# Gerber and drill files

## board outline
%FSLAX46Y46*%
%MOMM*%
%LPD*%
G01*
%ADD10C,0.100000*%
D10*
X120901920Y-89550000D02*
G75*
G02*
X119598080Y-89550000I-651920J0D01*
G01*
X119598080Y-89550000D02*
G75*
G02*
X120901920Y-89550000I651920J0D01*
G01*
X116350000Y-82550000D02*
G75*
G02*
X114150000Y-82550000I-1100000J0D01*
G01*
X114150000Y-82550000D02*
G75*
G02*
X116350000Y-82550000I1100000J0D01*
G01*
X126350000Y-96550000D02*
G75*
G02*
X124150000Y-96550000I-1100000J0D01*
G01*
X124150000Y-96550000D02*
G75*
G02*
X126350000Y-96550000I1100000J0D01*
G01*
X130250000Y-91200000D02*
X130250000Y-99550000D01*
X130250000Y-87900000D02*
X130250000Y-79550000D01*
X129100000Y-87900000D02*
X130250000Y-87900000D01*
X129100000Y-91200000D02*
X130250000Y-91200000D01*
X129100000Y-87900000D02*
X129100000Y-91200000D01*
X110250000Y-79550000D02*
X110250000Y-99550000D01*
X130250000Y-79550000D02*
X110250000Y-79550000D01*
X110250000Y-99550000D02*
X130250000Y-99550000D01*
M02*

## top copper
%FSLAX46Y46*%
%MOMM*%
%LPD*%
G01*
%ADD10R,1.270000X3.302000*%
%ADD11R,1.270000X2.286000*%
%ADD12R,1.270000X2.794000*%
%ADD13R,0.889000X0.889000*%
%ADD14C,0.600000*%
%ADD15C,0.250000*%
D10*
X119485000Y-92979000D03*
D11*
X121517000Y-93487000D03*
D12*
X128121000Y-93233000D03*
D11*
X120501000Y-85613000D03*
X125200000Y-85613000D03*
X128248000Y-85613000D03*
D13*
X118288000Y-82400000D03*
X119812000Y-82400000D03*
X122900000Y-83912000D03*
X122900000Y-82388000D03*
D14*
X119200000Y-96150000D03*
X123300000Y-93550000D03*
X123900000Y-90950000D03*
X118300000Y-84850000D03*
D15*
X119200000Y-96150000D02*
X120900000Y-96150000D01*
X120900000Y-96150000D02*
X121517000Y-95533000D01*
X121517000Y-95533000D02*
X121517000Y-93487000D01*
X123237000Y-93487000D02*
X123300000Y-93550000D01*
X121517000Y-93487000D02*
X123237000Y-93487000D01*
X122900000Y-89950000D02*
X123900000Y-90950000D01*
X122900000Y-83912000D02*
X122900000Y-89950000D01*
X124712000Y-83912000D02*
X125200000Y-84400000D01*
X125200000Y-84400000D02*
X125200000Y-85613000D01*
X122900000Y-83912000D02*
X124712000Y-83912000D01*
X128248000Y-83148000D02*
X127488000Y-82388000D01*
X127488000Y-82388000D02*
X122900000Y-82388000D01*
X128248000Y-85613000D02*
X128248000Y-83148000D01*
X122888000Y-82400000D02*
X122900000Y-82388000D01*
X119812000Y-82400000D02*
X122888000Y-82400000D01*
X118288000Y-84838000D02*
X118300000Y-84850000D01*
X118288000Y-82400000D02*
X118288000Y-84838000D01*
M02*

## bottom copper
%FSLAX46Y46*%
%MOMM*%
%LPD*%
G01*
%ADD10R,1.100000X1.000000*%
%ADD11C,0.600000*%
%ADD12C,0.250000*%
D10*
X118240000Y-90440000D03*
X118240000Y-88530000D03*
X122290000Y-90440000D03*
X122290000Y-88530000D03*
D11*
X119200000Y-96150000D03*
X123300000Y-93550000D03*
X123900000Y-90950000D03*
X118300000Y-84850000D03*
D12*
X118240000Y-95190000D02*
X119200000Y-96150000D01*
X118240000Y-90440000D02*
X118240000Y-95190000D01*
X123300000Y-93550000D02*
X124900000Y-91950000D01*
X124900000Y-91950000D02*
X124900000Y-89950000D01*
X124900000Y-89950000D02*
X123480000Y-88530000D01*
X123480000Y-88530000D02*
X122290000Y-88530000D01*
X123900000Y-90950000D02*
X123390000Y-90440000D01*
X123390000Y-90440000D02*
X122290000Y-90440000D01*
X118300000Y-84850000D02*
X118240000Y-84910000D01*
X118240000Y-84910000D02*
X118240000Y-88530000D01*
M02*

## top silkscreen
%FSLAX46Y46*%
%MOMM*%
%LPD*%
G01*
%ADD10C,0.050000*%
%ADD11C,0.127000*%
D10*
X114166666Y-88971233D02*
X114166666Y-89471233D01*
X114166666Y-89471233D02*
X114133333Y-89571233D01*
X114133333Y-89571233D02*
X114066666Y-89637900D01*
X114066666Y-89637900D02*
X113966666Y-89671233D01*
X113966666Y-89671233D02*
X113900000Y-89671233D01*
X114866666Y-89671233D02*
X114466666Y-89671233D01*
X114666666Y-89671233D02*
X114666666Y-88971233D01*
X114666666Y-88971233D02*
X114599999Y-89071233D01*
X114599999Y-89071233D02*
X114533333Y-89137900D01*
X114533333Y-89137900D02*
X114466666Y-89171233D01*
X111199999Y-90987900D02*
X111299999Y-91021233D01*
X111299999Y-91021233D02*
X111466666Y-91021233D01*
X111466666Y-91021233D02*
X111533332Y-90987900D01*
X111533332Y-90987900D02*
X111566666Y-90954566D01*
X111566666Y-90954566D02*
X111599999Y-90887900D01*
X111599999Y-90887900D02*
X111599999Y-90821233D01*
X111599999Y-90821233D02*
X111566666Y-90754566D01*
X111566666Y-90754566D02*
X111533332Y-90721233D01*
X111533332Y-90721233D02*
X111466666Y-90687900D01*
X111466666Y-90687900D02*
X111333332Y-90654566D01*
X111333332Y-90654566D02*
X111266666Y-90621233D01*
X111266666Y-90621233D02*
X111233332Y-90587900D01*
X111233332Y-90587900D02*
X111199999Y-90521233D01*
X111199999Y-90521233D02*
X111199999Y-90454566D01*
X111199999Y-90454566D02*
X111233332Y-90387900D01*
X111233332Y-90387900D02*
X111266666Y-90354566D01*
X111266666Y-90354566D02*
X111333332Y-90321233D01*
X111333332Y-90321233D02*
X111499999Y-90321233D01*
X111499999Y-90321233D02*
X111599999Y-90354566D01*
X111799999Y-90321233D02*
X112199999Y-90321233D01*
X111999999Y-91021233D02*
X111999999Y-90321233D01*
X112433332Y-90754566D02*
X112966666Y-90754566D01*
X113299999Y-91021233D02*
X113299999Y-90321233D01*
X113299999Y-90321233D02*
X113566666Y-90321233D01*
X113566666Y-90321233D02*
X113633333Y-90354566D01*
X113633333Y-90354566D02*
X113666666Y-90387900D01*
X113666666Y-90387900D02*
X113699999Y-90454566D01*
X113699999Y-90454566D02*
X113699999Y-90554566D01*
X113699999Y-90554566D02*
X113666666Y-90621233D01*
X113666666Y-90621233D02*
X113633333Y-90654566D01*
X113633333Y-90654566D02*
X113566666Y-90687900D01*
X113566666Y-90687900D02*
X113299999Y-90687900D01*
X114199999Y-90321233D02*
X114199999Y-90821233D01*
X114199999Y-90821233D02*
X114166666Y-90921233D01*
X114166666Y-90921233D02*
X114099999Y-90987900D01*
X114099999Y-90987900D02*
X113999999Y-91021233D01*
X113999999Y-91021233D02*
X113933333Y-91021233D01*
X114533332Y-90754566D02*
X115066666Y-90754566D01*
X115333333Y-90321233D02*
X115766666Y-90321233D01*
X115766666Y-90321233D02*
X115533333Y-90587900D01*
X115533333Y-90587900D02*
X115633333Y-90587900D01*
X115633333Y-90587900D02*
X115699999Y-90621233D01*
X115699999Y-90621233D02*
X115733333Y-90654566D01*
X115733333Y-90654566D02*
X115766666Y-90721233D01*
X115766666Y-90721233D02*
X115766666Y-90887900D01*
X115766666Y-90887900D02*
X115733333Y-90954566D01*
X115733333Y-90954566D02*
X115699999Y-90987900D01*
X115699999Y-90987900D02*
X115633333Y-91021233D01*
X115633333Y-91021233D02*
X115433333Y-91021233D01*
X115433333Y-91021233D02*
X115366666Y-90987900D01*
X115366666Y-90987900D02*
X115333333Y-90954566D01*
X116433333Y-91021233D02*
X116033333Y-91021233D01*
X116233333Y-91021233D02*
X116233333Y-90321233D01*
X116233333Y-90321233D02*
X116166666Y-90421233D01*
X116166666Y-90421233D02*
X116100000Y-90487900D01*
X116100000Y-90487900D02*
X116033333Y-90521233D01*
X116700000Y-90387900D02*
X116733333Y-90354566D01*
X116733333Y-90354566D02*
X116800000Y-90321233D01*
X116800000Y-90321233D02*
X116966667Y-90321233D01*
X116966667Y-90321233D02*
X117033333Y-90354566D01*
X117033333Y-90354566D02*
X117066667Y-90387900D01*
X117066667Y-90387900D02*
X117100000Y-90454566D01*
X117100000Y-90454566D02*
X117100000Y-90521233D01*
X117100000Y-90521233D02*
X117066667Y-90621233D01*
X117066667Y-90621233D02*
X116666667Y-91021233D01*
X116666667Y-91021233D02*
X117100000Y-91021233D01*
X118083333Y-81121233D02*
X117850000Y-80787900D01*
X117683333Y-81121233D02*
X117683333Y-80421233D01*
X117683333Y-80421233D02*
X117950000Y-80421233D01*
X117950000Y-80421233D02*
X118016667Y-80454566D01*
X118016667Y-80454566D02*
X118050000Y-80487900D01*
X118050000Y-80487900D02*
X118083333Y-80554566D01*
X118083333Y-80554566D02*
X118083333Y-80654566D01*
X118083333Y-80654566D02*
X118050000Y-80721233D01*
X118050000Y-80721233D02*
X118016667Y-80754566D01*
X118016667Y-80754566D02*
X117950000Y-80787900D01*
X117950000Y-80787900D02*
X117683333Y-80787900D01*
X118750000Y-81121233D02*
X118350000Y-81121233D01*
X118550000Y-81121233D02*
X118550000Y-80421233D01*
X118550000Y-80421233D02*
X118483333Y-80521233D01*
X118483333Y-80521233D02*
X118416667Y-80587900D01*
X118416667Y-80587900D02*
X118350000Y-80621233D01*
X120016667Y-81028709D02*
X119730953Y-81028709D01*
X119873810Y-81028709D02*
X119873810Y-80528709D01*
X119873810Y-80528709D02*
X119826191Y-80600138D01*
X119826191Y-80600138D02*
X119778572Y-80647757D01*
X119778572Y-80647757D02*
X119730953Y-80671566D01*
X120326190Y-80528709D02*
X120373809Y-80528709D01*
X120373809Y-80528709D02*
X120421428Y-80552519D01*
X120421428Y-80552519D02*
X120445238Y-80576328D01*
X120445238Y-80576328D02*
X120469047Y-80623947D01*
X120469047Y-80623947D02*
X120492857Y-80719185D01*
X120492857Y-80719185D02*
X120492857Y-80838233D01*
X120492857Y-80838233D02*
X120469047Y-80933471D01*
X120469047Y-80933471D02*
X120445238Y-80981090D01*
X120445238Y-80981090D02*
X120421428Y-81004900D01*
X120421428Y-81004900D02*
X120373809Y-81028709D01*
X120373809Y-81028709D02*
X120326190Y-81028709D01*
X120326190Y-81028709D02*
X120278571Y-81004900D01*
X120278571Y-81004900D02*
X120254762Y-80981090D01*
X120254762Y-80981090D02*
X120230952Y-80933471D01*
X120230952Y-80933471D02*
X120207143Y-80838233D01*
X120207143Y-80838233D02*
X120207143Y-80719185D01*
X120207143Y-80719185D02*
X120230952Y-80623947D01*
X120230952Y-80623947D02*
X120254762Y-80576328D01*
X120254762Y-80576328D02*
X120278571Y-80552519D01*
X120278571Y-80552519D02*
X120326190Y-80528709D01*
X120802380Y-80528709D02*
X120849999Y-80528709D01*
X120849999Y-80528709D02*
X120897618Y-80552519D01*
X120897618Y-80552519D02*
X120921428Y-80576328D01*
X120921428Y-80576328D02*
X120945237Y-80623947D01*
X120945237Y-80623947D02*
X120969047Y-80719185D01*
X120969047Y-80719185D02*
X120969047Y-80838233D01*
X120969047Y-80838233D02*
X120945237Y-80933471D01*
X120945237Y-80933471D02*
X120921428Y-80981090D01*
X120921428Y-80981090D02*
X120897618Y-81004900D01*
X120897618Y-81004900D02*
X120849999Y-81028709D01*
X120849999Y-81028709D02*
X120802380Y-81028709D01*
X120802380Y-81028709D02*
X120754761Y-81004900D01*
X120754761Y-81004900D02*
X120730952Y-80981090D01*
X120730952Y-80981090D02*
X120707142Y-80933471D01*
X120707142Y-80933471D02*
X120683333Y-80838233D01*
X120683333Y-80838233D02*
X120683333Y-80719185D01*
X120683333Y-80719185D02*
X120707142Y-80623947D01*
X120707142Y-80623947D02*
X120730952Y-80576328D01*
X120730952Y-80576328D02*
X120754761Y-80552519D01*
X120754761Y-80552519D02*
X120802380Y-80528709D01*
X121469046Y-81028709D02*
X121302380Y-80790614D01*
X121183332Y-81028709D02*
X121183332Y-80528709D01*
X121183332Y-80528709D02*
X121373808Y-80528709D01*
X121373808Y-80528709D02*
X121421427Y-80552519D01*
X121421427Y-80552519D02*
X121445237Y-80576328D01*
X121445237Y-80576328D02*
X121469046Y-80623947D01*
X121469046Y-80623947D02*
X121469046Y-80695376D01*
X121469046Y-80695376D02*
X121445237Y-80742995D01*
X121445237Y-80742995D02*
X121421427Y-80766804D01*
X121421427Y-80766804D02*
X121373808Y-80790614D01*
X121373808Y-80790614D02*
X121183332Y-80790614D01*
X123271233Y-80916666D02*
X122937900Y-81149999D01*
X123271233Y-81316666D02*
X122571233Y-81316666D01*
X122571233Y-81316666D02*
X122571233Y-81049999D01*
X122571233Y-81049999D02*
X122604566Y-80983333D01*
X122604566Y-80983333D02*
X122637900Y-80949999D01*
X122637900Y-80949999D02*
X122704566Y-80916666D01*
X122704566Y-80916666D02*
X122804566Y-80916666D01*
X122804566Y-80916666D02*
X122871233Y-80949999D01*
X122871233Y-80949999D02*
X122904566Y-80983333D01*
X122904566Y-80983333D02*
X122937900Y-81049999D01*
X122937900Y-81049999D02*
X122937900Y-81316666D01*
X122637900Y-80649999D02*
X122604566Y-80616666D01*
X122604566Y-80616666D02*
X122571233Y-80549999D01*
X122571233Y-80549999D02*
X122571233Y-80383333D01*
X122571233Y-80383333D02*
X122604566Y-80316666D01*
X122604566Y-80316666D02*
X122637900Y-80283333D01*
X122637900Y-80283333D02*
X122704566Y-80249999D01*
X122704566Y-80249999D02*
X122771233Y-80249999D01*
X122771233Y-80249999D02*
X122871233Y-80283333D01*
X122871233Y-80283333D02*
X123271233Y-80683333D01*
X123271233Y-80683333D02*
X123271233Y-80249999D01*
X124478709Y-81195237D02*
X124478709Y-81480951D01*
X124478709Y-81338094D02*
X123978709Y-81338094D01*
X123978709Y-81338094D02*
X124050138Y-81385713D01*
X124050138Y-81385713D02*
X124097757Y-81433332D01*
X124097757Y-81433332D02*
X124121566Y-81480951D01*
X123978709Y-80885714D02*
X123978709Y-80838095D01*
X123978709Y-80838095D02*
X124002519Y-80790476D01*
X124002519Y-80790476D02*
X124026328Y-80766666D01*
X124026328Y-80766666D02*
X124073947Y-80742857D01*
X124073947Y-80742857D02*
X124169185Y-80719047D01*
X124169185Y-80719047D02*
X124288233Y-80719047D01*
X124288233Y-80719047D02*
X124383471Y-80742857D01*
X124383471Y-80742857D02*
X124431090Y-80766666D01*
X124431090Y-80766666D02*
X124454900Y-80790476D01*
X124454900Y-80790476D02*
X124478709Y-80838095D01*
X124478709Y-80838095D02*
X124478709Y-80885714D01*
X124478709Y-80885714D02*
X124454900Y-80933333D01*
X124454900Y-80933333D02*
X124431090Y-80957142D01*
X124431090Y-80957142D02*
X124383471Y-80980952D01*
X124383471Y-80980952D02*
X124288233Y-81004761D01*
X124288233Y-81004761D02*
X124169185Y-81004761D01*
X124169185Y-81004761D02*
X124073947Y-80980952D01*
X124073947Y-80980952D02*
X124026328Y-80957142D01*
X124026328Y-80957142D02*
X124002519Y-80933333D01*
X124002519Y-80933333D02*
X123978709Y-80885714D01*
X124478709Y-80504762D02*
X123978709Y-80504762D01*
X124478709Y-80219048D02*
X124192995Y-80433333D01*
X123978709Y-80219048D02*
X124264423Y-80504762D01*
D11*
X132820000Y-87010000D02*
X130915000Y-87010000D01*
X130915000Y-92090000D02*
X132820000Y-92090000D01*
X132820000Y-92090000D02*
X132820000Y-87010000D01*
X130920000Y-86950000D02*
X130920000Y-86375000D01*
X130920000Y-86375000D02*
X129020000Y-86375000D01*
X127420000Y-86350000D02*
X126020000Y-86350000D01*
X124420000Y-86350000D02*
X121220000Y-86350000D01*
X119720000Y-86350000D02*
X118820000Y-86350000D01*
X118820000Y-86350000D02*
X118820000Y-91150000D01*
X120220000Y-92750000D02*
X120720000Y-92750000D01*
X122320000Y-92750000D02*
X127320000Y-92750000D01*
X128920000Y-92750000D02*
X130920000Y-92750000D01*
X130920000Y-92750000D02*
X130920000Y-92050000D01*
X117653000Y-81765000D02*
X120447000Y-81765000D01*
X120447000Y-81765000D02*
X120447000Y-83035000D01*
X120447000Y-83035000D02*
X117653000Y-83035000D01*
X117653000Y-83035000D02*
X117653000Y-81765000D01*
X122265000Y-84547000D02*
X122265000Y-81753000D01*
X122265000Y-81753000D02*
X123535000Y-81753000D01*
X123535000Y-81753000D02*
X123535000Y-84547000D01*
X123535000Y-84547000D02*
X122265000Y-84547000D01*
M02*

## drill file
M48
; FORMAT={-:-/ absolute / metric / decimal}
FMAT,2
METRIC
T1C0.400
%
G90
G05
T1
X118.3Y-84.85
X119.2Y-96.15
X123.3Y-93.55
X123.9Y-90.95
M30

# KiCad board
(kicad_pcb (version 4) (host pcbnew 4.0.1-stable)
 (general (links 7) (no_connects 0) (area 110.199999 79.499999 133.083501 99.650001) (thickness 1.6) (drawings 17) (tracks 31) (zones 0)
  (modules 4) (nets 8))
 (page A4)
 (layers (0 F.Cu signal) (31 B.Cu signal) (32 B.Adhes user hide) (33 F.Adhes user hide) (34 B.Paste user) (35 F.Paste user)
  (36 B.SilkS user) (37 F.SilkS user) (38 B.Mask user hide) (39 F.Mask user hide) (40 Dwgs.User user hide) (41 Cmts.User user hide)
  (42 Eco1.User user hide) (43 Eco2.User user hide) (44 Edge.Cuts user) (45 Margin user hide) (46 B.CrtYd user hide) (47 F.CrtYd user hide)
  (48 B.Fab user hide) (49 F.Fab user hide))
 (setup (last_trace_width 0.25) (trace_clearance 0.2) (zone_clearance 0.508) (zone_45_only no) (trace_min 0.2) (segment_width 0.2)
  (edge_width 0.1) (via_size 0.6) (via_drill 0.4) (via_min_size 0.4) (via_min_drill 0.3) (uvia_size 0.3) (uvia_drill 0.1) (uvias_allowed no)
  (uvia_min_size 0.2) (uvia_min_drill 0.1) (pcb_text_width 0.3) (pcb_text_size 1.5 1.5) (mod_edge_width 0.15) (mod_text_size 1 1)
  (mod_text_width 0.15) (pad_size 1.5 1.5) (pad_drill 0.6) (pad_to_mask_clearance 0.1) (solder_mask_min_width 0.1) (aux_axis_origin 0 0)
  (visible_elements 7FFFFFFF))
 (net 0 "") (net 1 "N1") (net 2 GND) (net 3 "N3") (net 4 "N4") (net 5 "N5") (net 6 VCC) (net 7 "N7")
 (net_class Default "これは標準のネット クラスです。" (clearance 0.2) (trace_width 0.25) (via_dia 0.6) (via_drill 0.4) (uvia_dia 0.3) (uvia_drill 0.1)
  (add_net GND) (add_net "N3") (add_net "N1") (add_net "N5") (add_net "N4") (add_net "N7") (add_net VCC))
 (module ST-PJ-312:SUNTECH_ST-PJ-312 (layer F.Cu) (at 125.2 89.55) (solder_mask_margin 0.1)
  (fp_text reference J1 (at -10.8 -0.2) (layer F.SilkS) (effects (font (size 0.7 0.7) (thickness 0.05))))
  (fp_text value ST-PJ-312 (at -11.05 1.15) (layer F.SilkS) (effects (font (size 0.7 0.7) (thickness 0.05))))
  (fp_line (start 7.62 -2.54) (end 5.715 -2.54) (layer F.SilkS) (width 0.127))
  (fp_line (start 5.715 2.54) (end 7.62 2.54) (layer F.SilkS) (width 0.127))
  (fp_line (start 7.62 2.54) (end 7.62 -2.54) (layer F.SilkS) (width 0.127))
  (fp_line (start 5.72 -2.6) (end 5.72 -3.175) (layer F.SilkS) (width 0.127))
  (fp_line (start 5.72 -3.175) (end 3.82 -3.175) (layer F.SilkS) (width 0.127))
  (fp_line (start 2.22 -3.2) (end 0.82 -3.2) (layer F.SilkS) (width 0.127))
  (fp_line (start -0.78 -3.2) (end -3.98 -3.2) (layer F.SilkS) (width 0.127))
  (fp_line (start -5.48 -3.2) (end -6.38 -3.2) (layer F.SilkS) (width 0.127))
  (fp_line (start -6.38 -3.2) (end -6.38 1.6) (layer F.SilkS) (width 0.127))
  (fp_line (start -4.98 3.2) (end -4.48 3.2) (layer F.SilkS) (width 0.127))
  (fp_line (start -2.88 3.2) (end 2.12 3.2) (layer F.SilkS) (width 0.127))
  (fp_line (start 3.72 3.2) (end 5.72 3.2) (layer F.SilkS) (width 0.127))
  (fp_line (start 5.72 3.2) (end 5.72 2.5) (layer F.SilkS) (width 0.127))
  (pad LS smd rect (at -5.715 3.429 90) (size 3.302 1.27) (layers F.Cu F.Paste F.Mask) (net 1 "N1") (solder_mask_margin 0.2))
  (pad L smd rect (at -3.683 3.937 90) (size 2.286 1.27) (layers F.Cu F.Paste F.Mask) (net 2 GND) (solder_mask_margin 0.2))
  (pad COM2 smd rect (at 2.921 3.683 90) (size 2.794 1.27) (layers F.Cu F.Paste F.Mask) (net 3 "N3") (solder_mask_margin 0.2))
  (pad RS smd rect (at -4.699 -3.937 90) (size 2.286 1.27) (layers F.Cu F.Paste F.Mask) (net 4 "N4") (solder_mask_margin 0.2))
  (pad R smd rect (at 0 -3.937 90) (size 2.286 1.27) (layers F.Cu F.Paste F.Mask) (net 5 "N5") (solder_mask_margin 0.2))
  (pad COM1 smd rect (at 3.048 -3.937 90) (size 2.286 1.27) (layers F.Cu F.Paste F.Mask) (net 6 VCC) (solder_mask_margin 0.2)))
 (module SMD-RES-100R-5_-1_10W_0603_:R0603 (layer F.Cu) (at 119.05 82.4 90) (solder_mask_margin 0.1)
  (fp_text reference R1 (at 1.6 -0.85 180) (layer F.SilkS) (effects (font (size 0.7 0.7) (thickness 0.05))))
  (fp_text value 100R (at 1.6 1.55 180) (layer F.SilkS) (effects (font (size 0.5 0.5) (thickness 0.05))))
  (fp_line (start 0.635 -1.397) (end 0.635 1.397) (layer F.SilkS) (width 0.127))
  (fp_line (start 0.635 1.397) (end -0.635 1.397) (layer F.SilkS) (width 0.127))
  (fp_line (start -0.635 1.397) (end -0.635 -1.397) (layer F.SilkS) (width 0.127))
  (fp_line (start -0.635 -1.397) (end 0.635 -1.397) (layer F.SilkS) (width 0.127))
  (pad 1 smd rect (at 0 -0.762) (size 0.889 0.889) (layers F.Cu F.Paste F.Mask) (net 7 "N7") (solder_mask_margin 0.2))
  (pad 2 smd rect (at 0 0.762) (size 0.889 0.889) (layers F.Cu F.Paste F.Mask) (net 6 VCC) (solder_mask_margin 0.2)))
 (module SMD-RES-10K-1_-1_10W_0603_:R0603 (layer F.Cu) (at 122.9 83.15 180) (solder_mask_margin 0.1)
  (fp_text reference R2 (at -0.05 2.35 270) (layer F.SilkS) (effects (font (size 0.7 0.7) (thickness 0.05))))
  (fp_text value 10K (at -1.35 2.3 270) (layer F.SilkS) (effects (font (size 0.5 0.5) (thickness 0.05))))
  (fp_line (start 0.635 -1.397) (end 0.635 1.397) (layer F.SilkS) (width 0.127))
  (fp_line (start 0.635 1.397) (end -0.635 1.397) (layer F.SilkS) (width 0.127))
  (fp_line (start -0.635 1.397) (end -0.635 -1.397) (layer F.SilkS) (width 0.127))
  (fp_line (start -0.635 -1.397) (end 0.635 -1.397) (layer F.SilkS) (width 0.127))
  (pad 1 smd rect (at 0 -0.762 90) (size 0.889 0.889) (layers F.Cu F.Paste F.Mask) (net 5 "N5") (solder_mask_margin 0.2))
  (pad 2 smd rect (at 0 0.762 90) (size 0.889 0.889) (layers F.Cu F.Paste F.Mask) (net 6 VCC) (solder_mask_margin 0.2)))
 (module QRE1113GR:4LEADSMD (layer B.Cu) (at 120.25 89.5) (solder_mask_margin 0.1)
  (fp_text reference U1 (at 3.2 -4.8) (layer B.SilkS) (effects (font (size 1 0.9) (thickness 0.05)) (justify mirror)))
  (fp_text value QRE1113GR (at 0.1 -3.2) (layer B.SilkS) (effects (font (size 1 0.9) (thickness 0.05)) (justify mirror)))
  (pad E smd rect (at -2.01 0.94 90) (size 1 1.1) (layers B.Cu B.Paste B.Mask) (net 2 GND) (solder_mask_margin 0.2))
  (pad A smd rect (at -2.01 -0.97 90) (size 1 1.1) (layers B.Cu B.Paste B.Mask) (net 7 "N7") (solder_mask_margin 0.2))
  (pad C smd rect (at 2.04 0.94 90) (size 1 1.1) (layers B.Cu B.Paste B.Mask) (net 5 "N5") (solder_mask_margin 0.2))
  (pad K smd rect (at 2.04 -0.97 90) (size 1 1.1) (layers B.Cu B.Paste B.Mask) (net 2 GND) (solder_mask_margin 0.2)))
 (gr_circle (center 120.25 89.55) (end 120.3 88.9) (layer Edge.Cuts) (width 0.1))
 (gr_circle (center 115.25 82.55) (end 116.35 82.55) (layer Edge.Cuts) (width 0.1))
 (gr_circle (center 125.25 96.55) (end 126.35 96.55) (layer Edge.Cuts) (width 0.1))
 (gr_line (start 130.25 91.2) (end 130.25 99.55) (angle 90) (layer Edge.Cuts) (width 0.1))
 (gr_line (start 130.25 87.9) (end 130.25 79.55) (angle 90) (layer Edge.Cuts) (width 0.1))
 (gr_line (start 129.1 87.9) (end 130.25 87.9) (angle 90) (layer Edge.Cuts) (width 0.1))
 (gr_line (start 129.1 91.2) (end 130.25 91.2) (angle 90) (layer Edge.Cuts) (width 0.1))
 (gr_line (start 129.1 87.9) (end 129.1 91.2) (angle 90) (layer Edge.Cuts) (width 0.1))
 (gr_line (start 110.25 79.55) (end 110.25 99.55) (angle 90) (layer Edge.Cuts) (width 0.1))
 (gr_line (start 130.25 79.55) (end 110.25 79.55) (angle 90) (layer Edge.Cuts) (width 0.1))
 (gr_line (start 110.25 99.55) (end 130.25 99.55) (angle 90) (layer Edge.Cuts) (width 0.1))
 (segment (start 118.24 95.19) (end 119.2 96.15) (width 0.25) (layer B.Cu) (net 2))
 (via (at 119.2 96.15) (size 0.6) (layers F.Cu B.Cu) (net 2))
 (segment (start 119.2 96.15) (end 120.9 96.15) (width 0.25) (layer F.Cu) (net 2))
 (segment (start 120.9 96.15) (end 121.517 95.533) (width 0.25) (layer F.Cu) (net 2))
 (segment (start 121.517 95.533) (end 121.517 93.487) (width 0.25) (layer F.Cu) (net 2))
 (segment (start 118.24 90.44) (end 118.24 95.19) (width 0.25) (layer B.Cu) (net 2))
 (segment (start 123.237 93.487) (end 123.3 93.55) (width 0.25) (layer F.Cu) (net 2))
 (via (at 123.3 93.55) (size 0.6) (layers F.Cu B.Cu) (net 2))
 (segment (start 123.3 93.55) (end 124.9 91.95) (width 0.25) (layer B.Cu) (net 2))
 (segment (start 124.9 91.95) (end 124.9 89.95) (width 0.25) (layer B.Cu) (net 2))
 (segment (start 124.9 89.95) (end 123.48 88.53) (width 0.25) (layer B.Cu) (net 2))
 (segment (start 123.48 88.53) (end 122.29 88.53) (width 0.25) (layer B.Cu) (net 2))
 (segment (start 121.517 93.487) (end 123.237 93.487) (width 0.25) (layer F.Cu) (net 2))
 (segment (start 122.9 89.95) (end 123.9 90.95) (width 0.25) (layer F.Cu) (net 5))
 (via (at 123.9 90.95) (size 0.6) (layers F.Cu B.Cu) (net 5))
 (segment (start 123.9 90.95) (end 123.39 90.44) (width 0.25) (layer B.Cu) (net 5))
 (segment (start 123.39 90.44) (end 122.29 90.44) (width 0.25) (layer B.Cu) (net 5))
 (segment (start 122.9 83.912) (end 122.9 89.95) (width 0.25) (layer F.Cu) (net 5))
 (segment (start 124.712 83.912) (end 125.2 84.4) (width 0.25) (layer F.Cu) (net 5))
 (segment (start 125.2 84.4) (end 125.2 85.613) (width 0.25) (layer F.Cu) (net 5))
 (segment (start 122.9 83.912) (end 124.712 83.912) (width 0.25) (layer F.Cu) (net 5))
 (segment (start 128.248 83.148) (end 127.488 82.388) (width 0.25) (layer F.Cu) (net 6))
 (segment (start 127.488 82.388) (end 122.9 82.388) (width 0.25) (layer F.Cu) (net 6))
 (segment (start 128.248 85.613) (end 128.248 83.148) (width 0.25) (layer F.Cu) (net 6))
 (segment (start 122.888 82.4) (end 122.9 82.388) (width 0.25) (layer F.Cu) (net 6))
 (segment (start 119.812 82.4) (end 122.888 82.4) (width 0.25) (layer F.Cu) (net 6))
 (segment (start 118.288 84.838) (end 118.3 84.85) (width 0.25) (layer F.Cu) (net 7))
 (via (at 118.3 84.85) (size 0.6) (layers F.Cu B.Cu) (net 7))
 (segment (start 118.3 84.85) (end 118.24 84.91) (width 0.25) (layer B.Cu) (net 7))
 (segment (start 118.24 84.91) (end 118.24 88.53) (width 0.25) (layer B.Cu) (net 7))
 (segment (start 118.288 82.4) (end 118.288 84.838) (width 0.25) (layer F.Cu) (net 7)))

